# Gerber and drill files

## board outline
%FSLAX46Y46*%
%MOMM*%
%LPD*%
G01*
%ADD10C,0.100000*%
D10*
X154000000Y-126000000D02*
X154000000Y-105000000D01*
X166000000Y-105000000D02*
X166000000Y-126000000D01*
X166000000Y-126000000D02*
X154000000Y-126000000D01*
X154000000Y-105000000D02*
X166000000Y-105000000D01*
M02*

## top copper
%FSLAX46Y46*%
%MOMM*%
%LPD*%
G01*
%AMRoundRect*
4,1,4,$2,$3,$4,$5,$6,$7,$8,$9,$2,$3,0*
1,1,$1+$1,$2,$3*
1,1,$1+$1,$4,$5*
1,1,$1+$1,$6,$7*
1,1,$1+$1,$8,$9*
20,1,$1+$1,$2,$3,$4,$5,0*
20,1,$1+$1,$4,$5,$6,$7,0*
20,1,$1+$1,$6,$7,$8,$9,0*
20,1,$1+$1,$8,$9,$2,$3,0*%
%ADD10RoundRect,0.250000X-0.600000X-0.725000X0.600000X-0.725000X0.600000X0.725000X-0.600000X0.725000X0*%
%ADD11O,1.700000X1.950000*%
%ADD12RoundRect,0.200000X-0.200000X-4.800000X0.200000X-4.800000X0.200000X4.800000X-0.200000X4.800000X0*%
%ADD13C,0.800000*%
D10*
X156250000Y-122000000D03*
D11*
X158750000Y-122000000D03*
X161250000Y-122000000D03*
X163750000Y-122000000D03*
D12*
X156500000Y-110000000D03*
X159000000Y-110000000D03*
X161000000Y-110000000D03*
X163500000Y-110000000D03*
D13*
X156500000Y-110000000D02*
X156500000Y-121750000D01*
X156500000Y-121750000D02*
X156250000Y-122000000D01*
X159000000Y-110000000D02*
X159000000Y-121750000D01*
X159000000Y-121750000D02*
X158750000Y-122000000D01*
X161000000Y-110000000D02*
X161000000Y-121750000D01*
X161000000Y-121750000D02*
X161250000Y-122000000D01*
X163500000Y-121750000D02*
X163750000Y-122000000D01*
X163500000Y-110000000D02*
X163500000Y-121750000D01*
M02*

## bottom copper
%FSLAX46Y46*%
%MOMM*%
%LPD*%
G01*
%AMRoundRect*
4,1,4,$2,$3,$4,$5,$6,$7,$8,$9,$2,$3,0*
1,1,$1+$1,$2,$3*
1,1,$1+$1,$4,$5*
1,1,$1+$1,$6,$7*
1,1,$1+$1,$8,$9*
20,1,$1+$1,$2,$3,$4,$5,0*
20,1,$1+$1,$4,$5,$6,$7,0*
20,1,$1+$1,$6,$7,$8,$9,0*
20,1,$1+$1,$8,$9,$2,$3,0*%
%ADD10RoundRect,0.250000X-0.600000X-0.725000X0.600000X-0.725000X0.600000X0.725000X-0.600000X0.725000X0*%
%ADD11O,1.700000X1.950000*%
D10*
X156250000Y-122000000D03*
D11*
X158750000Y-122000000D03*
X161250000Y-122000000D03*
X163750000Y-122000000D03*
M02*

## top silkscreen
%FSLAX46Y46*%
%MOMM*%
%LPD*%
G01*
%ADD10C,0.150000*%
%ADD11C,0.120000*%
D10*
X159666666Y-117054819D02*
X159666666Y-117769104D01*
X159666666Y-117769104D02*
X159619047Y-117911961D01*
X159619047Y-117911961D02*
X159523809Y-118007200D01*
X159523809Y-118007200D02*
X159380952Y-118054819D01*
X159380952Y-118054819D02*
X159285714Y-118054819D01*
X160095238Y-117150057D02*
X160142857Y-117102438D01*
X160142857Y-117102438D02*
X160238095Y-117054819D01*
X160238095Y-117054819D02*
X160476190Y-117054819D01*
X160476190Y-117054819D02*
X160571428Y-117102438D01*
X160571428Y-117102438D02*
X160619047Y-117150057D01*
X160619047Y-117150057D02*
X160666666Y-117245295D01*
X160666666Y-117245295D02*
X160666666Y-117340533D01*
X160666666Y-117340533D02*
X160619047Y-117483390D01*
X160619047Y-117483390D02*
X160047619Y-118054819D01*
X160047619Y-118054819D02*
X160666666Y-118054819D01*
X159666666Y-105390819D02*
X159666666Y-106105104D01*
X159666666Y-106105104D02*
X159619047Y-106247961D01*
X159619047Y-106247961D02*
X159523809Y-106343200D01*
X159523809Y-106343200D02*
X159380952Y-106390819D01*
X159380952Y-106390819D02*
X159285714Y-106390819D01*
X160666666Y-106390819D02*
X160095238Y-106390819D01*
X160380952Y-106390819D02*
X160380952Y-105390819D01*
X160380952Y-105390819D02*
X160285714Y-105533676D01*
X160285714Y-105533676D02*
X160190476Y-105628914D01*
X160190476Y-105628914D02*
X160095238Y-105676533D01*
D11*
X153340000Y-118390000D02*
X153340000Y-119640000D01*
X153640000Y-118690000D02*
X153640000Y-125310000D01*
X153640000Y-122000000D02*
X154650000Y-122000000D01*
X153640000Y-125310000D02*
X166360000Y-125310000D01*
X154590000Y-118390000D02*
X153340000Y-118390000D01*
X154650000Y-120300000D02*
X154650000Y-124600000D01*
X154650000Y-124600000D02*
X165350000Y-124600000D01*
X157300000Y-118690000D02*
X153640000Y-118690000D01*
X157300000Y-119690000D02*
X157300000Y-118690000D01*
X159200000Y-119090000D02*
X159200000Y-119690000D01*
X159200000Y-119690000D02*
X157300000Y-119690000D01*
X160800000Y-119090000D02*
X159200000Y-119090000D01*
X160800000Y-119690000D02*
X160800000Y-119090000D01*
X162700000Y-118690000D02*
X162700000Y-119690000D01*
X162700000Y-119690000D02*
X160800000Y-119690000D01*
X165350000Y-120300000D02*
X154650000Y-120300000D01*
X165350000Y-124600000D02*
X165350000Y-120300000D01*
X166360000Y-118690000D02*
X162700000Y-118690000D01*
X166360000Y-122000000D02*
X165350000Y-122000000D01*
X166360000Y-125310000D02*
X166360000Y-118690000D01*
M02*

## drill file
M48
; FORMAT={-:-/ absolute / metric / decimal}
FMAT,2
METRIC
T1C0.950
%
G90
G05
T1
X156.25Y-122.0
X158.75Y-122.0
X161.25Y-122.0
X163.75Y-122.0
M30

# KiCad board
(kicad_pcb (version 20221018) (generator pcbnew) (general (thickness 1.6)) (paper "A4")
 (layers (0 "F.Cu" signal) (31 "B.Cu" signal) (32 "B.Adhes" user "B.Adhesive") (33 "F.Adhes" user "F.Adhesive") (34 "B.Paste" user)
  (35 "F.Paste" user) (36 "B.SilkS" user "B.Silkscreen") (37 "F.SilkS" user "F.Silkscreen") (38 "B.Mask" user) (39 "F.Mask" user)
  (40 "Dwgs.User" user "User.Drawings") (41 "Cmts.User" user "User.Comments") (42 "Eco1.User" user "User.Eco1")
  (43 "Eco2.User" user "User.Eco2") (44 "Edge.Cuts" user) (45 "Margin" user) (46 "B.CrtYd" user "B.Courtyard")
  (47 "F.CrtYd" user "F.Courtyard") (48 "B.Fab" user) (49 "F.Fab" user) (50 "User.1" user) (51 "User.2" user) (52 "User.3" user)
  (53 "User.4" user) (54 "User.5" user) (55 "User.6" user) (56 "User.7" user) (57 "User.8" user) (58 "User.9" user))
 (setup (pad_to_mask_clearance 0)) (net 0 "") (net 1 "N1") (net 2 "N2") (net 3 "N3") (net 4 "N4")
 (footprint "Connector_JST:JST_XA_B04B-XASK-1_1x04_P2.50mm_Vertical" (layer "F.Cu") (at 156.25 122)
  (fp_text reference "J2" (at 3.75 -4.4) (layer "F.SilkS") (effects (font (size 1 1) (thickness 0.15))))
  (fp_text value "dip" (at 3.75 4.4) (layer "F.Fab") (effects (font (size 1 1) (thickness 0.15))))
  (fp_line (start -2.91 -3.61) (end -2.91 -2.36) (stroke (width 0.12) (type solid)) (layer "F.SilkS"))
  (fp_line (start -2.61 -3.31) (end -2.61 3.31) (stroke (width 0.12) (type solid)) (layer "F.SilkS"))
  (fp_line (start -2.61 0) (end -1.6 0) (stroke (width 0.12) (type solid)) (layer "F.SilkS"))
  (fp_line (start -2.61 3.31) (end 10.11 3.31) (stroke (width 0.12) (type solid)) (layer "F.SilkS"))
  (fp_line (start -1.66 -3.61) (end -2.91 -3.61) (stroke (width 0.12) (type solid)) (layer "F.SilkS"))
  (fp_line (start -1.6 -1.7) (end -1.6 2.6) (stroke (width 0.12) (type solid)) (layer "F.SilkS"))
  (fp_line (start -1.6 2.6) (end 9.1 2.6) (stroke (width 0.12) (type solid)) (layer "F.SilkS"))
  (fp_line (start 1.05 -3.31) (end -2.61 -3.31) (stroke (width 0.12) (type solid)) (layer "F.SilkS"))
  (fp_line (start 1.05 -2.31) (end 1.05 -3.31) (stroke (width 0.12) (type solid)) (layer "F.SilkS"))
  (fp_line (start 2.95 -2.91) (end 2.95 -2.31) (stroke (width 0.12) (type solid)) (layer "F.SilkS"))
  (fp_line (start 2.95 -2.31) (end 1.05 -2.31) (stroke (width 0.12) (type solid)) (layer "F.SilkS"))
  (fp_line (start 4.55 -2.91) (end 2.95 -2.91) (stroke (width 0.12) (type solid)) (layer "F.SilkS"))
  (fp_line (start 4.55 -2.31) (end 4.55 -2.91) (stroke (width 0.12) (type solid)) (layer "F.SilkS"))
  (fp_line (start 6.45 -3.31) (end 6.45 -2.31) (stroke (width 0.12) (type solid)) (layer "F.SilkS"))
  (fp_line (start 6.45 -2.31) (end 4.55 -2.31) (stroke (width 0.12) (type solid)) (layer "F.SilkS"))
  (fp_line (start 9.1 -1.7) (end -1.6 -1.7) (stroke (width 0.12) (type solid)) (layer "F.SilkS"))
  (fp_line (start 9.1 2.6) (end 9.1 -1.7) (stroke (width 0.12) (type solid)) (layer "F.SilkS"))
  (fp_line (start 10.11 -3.31) (end 6.45 -3.31) (stroke (width 0.12) (type solid)) (layer "F.SilkS"))
  (fp_line (start 10.11 0) (end 9.1 0) (stroke (width 0.12) (type solid)) (layer "F.SilkS"))
  (fp_line (start 10.11 3.31) (end 10.11 -3.31) (stroke (width 0.12) (type solid)) (layer "F.SilkS"))
  (pad "1" thru_hole roundrect (at 0 0) (size 1.7 1.95) (drill 0.95) (layers "*.Cu" "*.Mask") (roundrect_rratio 0.147059) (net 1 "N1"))
  (pad "2" thru_hole oval (at 2.5 0) (size 1.7 1.95) (drill 0.95) (layers "*.Cu" "*.Mask") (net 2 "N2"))
  (pad "3" thru_hole oval (at 5 0) (size 1.7 1.95) (drill 0.95) (layers "*.Cu" "*.Mask") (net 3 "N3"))
  (pad "4" thru_hole oval (at 7.5 0) (size 1.7 1.95) (drill 0.95) (layers "*.Cu" "*.Mask") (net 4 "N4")))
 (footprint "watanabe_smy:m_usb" (layer "F.Cu") (at 160 110)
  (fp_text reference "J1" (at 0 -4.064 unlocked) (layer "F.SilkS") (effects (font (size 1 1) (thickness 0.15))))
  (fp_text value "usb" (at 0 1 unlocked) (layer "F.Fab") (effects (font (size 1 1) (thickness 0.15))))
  (pad "1" smd roundrect (at -3.5 0) (size 0.8 10) (layers "F.Cu" "F.Paste" "F.Mask") (roundrect_rratio 0.25) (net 1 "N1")
   (thermal_bridge_angle 45))
  (pad "2" smd roundrect (at -1 0) (size 0.8 10) (layers "*.Mask" "F.Cu" "F.Paste") (roundrect_rratio 0.25) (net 2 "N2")
   (thermal_bridge_angle 45))
  (pad "3" smd roundrect (at 1 0) (size 0.8 10) (layers "F.Cu" "F.Paste" "F.Mask") (roundrect_rratio 0.25) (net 3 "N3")
   (thermal_bridge_angle 45))
  (pad "4" smd roundrect (at 3.5 0) (size 0.8 10) (layers "F.Cu" "F.Paste" "F.Mask") (roundrect_rratio 0.25) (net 4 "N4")
   (thermal_bridge_angle 45)))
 (gr_line (start 154 126) (end 154 105) (stroke (width 0.1) (type default)) (layer "Edge.Cuts"))
 (gr_line (start 166 105) (end 166 126) (stroke (width 0.1) (type default)) (layer "Edge.Cuts"))
 (gr_line (start 166 126) (end 154 126) (stroke (width 0.1) (type default)) (layer "Edge.Cuts"))
 (gr_line (start 154 105) (end 166 105) (stroke (width 0.1) (type default)) (layer "Edge.Cuts"))
 (segment (start 156.5 110) (end 156.5 121.75) (width 0.8) (layer "F.Cu") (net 1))
 (segment (start 156.5 121.75) (end 156.25 122) (width 0.8) (layer "F.Cu") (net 1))
 (segment (start 159 110) (end 159 121.75) (width 0.8) (layer "F.Cu") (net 2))
 (segment (start 159 121.75) (end 158.75 122) (width 0.8) (layer "F.Cu") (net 2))
 (segment (start 161 110) (end 161 121.75) (width 0.8) (layer "F.Cu") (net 3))
 (segment (start 161 121.75) (end 161.25 122) (width 0.8) (layer "F.Cu") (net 3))
 (segment (start 163.5 121.75) (end 163.75 122) (width 0.8) (layer "F.Cu") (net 4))
 (segment (start 163.5 110) (end 163.5 121.75) (width 0.8) (layer "F.Cu") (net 4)))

